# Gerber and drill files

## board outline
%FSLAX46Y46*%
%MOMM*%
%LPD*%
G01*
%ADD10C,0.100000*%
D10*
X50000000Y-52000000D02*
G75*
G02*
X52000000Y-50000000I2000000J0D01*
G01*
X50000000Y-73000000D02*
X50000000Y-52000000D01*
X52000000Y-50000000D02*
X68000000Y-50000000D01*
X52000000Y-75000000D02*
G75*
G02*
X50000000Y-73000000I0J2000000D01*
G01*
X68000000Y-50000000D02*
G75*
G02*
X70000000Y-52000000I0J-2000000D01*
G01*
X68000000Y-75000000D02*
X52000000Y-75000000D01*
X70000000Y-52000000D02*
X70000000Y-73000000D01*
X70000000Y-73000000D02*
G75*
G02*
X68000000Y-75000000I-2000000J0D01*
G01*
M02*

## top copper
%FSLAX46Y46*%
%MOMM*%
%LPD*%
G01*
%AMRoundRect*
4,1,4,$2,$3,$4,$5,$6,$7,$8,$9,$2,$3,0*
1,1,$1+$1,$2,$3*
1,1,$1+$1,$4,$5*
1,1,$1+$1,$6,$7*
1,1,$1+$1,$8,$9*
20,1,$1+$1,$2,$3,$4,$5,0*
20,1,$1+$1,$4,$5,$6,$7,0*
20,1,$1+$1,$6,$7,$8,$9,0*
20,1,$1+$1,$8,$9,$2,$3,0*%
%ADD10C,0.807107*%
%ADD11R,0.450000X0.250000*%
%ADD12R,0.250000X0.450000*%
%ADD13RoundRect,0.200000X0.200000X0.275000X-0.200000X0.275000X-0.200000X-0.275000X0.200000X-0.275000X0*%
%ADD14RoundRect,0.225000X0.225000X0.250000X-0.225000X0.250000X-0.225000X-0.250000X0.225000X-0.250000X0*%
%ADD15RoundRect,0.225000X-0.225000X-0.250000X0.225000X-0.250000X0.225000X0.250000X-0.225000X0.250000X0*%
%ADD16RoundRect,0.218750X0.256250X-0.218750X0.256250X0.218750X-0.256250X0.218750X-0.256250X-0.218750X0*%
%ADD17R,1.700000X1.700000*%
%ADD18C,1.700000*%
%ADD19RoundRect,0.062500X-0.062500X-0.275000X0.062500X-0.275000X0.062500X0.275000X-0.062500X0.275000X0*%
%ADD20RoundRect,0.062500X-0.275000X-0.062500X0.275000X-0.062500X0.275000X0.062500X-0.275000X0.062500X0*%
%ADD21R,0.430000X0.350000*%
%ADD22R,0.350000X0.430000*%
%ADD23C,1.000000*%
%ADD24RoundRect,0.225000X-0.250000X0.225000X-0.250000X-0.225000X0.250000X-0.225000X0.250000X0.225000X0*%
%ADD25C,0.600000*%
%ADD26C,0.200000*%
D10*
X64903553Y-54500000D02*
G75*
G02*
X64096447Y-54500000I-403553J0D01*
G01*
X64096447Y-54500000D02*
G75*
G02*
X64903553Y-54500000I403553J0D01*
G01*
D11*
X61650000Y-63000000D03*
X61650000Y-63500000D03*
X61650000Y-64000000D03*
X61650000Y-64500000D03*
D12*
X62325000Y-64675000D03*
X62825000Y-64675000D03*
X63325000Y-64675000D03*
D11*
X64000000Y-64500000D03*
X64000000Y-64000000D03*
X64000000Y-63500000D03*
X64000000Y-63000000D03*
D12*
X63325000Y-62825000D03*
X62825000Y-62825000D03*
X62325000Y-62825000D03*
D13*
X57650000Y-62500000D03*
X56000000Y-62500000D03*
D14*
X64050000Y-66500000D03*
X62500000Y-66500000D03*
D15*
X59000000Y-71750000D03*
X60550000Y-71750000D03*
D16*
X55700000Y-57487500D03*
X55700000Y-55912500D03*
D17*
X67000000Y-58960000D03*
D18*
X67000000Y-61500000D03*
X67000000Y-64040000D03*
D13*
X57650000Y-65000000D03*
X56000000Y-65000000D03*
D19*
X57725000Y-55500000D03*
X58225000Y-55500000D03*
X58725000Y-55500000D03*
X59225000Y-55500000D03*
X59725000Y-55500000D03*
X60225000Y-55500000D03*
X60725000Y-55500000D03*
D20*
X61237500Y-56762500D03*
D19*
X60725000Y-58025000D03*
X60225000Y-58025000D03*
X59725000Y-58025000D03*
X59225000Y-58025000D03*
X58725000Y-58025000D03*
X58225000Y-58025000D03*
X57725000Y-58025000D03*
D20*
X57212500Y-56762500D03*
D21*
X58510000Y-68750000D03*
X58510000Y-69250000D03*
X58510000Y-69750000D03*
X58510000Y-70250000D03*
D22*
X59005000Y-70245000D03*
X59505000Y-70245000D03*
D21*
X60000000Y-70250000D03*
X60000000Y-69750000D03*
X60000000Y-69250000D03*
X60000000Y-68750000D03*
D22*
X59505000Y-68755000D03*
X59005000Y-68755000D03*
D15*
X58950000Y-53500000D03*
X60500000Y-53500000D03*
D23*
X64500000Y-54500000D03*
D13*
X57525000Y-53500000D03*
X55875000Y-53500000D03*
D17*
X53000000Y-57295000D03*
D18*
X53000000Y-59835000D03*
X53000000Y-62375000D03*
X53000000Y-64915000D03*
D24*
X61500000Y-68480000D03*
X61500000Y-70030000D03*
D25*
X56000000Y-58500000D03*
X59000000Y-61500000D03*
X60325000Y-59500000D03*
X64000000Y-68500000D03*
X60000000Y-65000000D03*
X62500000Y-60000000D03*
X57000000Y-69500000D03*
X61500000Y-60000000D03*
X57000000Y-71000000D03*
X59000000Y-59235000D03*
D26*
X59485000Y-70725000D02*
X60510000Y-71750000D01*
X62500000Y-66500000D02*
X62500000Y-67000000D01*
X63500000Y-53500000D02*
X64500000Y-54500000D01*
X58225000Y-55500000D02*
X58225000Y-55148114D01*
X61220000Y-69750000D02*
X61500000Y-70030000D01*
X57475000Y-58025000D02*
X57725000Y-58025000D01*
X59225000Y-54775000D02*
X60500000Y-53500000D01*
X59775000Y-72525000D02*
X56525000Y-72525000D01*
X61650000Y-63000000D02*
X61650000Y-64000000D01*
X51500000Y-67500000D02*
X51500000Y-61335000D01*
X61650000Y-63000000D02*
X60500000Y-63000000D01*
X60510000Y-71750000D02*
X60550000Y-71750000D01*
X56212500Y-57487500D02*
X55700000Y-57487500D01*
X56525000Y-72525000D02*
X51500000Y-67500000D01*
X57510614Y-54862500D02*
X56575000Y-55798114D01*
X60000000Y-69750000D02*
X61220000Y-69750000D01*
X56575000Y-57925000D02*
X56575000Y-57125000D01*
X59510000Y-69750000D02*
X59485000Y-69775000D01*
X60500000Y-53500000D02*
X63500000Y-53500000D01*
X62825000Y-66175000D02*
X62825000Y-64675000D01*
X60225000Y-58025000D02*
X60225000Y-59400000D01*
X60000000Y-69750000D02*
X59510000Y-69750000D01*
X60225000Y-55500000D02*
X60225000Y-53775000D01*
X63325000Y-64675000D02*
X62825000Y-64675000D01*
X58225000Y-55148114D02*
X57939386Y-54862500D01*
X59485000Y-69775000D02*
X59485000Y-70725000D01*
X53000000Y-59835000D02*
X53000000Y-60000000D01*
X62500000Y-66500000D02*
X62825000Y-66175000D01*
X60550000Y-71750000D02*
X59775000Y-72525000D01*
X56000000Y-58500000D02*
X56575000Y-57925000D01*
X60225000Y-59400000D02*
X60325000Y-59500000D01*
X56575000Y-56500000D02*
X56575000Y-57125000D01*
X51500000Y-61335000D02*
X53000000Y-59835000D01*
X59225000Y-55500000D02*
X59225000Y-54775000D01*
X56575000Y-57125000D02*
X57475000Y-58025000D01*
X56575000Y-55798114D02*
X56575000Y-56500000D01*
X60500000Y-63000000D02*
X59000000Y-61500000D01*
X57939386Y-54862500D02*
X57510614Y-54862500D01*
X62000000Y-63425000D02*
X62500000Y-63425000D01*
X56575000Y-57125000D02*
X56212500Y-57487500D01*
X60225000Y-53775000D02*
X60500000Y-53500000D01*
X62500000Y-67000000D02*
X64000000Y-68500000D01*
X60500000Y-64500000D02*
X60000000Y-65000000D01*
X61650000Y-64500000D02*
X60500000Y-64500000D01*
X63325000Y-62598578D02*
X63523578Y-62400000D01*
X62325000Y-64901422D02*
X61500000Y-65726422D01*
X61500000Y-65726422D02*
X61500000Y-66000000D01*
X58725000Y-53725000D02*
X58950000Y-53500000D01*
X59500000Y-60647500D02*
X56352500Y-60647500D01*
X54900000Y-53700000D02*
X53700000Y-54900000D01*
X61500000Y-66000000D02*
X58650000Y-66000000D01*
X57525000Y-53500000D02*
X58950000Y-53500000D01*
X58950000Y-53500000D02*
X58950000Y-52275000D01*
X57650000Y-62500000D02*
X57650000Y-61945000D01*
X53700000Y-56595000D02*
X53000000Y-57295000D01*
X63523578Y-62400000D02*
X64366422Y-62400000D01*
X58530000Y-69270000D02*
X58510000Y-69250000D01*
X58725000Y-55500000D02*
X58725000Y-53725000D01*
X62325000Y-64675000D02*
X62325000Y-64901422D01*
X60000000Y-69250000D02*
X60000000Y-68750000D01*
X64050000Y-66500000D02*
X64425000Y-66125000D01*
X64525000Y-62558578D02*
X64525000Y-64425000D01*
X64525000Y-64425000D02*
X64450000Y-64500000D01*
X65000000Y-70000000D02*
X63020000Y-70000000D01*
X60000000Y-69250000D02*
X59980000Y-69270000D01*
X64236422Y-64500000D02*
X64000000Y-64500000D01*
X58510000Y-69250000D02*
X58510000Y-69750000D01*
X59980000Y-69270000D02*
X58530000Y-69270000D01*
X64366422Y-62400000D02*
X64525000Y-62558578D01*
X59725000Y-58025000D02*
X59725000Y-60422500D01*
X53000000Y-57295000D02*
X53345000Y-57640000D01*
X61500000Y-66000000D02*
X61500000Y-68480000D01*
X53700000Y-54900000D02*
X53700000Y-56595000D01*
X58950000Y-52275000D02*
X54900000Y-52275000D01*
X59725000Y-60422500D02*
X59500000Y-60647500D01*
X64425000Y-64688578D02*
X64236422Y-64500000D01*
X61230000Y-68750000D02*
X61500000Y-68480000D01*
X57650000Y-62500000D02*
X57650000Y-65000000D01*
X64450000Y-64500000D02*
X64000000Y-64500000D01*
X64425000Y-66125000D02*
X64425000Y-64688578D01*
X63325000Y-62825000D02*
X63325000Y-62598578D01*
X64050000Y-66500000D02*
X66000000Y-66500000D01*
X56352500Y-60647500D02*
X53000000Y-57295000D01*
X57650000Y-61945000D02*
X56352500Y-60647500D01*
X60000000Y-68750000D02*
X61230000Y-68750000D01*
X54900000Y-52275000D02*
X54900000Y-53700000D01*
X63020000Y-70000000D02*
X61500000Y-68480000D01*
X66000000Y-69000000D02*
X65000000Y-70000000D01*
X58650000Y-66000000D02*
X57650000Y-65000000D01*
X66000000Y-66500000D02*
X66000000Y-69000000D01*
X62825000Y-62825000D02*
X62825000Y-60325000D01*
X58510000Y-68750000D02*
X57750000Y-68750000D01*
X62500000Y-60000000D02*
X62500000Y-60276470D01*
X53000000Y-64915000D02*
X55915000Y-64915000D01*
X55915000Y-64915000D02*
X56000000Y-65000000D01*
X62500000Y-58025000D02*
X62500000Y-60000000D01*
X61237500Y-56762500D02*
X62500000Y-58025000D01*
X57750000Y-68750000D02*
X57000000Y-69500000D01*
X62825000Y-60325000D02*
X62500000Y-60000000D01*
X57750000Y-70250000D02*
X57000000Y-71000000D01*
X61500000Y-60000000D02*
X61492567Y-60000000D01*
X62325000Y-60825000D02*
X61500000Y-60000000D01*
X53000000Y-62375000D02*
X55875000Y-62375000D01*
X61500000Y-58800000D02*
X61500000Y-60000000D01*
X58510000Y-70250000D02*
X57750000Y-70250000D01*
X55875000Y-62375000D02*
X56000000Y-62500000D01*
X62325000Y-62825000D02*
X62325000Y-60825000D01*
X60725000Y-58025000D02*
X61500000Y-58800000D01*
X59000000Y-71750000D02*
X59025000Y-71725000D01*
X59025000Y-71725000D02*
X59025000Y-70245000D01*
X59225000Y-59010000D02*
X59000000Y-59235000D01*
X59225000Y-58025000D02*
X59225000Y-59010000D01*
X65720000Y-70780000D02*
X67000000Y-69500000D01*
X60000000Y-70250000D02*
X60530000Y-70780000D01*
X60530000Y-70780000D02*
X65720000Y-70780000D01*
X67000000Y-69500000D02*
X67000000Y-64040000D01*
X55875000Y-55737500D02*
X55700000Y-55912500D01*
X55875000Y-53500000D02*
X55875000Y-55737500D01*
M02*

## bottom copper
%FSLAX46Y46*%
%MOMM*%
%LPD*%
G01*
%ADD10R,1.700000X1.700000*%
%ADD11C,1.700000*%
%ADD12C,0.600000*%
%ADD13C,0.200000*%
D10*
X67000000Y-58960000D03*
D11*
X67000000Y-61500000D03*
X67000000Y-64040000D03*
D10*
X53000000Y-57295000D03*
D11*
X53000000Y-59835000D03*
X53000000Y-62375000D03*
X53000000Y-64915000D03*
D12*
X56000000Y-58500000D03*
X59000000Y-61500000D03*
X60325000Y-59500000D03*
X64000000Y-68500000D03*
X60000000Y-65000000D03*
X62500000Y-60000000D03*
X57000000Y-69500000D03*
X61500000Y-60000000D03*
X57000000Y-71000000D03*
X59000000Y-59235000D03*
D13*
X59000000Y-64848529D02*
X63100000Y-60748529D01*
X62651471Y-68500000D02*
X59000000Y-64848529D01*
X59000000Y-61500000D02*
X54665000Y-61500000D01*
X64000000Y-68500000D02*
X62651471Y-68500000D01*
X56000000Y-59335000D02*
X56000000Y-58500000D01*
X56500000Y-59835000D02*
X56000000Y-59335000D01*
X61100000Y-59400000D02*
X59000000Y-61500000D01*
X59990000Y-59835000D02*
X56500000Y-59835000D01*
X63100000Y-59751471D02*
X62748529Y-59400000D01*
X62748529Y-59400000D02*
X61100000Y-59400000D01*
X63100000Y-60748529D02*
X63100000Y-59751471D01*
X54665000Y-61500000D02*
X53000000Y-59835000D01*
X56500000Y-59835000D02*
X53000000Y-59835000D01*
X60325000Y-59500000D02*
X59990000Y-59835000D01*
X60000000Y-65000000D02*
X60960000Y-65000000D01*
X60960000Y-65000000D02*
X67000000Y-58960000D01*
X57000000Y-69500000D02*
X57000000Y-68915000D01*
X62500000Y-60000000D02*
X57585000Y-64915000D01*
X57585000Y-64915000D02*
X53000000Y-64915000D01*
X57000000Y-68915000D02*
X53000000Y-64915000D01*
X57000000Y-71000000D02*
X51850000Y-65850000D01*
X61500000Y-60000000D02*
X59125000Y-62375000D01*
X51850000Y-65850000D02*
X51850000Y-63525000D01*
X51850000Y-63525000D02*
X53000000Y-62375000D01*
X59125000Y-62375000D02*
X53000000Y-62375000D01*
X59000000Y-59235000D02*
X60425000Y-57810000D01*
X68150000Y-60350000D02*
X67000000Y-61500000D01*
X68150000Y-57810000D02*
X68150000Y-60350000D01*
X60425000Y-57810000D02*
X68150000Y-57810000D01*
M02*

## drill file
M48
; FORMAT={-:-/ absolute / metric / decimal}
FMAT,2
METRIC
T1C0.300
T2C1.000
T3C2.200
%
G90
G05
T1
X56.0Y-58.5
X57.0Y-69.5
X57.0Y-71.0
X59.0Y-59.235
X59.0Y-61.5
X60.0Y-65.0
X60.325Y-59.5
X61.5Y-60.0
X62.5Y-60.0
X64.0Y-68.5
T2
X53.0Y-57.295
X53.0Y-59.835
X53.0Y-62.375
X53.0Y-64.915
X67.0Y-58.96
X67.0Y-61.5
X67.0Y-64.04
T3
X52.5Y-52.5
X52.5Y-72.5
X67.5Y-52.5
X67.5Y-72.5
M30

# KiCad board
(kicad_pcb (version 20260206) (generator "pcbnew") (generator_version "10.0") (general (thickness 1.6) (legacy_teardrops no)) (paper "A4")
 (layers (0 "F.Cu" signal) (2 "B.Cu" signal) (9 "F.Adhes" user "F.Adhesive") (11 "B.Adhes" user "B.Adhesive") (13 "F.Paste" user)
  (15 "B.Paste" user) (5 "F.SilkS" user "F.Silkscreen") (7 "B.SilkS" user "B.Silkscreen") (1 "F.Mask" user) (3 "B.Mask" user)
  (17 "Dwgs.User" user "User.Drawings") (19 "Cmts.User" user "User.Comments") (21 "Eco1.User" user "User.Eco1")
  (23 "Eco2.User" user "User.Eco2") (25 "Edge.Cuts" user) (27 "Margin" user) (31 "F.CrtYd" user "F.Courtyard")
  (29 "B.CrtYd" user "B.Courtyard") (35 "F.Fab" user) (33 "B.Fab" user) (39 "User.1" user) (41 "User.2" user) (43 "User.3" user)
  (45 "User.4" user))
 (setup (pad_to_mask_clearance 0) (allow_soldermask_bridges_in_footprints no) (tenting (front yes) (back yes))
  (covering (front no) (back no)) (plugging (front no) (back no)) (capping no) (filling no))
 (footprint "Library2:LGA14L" (layer "F.Cu") (at 62.825 63.75)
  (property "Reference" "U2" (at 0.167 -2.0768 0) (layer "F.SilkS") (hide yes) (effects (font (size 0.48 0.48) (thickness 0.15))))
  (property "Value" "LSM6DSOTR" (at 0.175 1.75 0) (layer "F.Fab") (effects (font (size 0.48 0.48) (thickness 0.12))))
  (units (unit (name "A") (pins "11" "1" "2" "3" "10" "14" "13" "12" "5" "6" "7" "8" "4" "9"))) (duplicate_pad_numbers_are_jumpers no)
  (pad "1" smd rect (at -1.175 -0.75) (size 0.45 0.25) (layers "F.Cu" "F.Mask" "F.Paste") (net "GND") (solder_mask_margin 0.102))
  (pad "2" smd rect (at -1.175 -0.25) (size 0.45 0.25) (layers "F.Cu" "F.Mask" "F.Paste") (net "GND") (solder_mask_margin 0.102))
  (pad "3" smd rect (at -1.175 0.25) (size 0.45 0.25) (layers "F.Cu" "F.Mask" "F.Paste") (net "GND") (solder_mask_margin 0.102))
  (pad "4" smd rect (at -1.175 0.75) (size 0.45 0.25) (layers "F.Cu" "F.Mask" "F.Paste") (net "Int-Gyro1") (solder_mask_margin 0.102))
  (pad "5" smd rect (at -0.5 0.925) (size 0.25 0.45) (layers "F.Cu" "F.Mask" "F.Paste") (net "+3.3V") (solder_mask_margin 0.102))
  (pad "6" smd rect (at 0 0.925) (size 0.25 0.45) (layers "F.Cu" "F.Mask" "F.Paste") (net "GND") (solder_mask_margin 0.102))
  (pad "7" smd rect (at 0.5 0.925) (size 0.25 0.45) (layers "F.Cu" "F.Mask" "F.Paste") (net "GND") (solder_mask_margin 0.102))
  (pad "8" smd rect (at 1.175 0.75) (size 0.45 0.25) (layers "F.Cu" "F.Mask" "F.Paste") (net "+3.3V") (solder_mask_margin 0.102))
  (pad "9" smd rect (at 1.175 0.25) (size 0.45 0.25) (layers "F.Cu" "F.Mask" "F.Paste") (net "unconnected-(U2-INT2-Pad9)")
   (solder_mask_margin 0.102))
  (pad "10" smd rect (at 1.175 -0.25) (size 0.45 0.25) (layers "F.Cu" "F.Mask" "F.Paste") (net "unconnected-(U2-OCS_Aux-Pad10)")
   (solder_mask_margin 0.102))
  (pad "11" smd rect (at 1.175 -0.75) (size 0.45 0.25) (layers "F.Cu" "F.Mask" "F.Paste") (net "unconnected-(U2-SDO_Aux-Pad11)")
   (solder_mask_margin 0.102))
  (pad "12" smd rect (at 0.5 -0.925) (size 0.25 0.45) (layers "F.Cu" "F.Mask" "F.Paste") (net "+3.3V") (solder_mask_margin 0.102))
  (pad "13" smd rect (at 0 -0.925) (size 0.25 0.45) (layers "F.Cu" "F.Mask" "F.Paste") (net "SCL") (solder_mask_margin 0.102))
  (pad "14" smd rect (at -0.5 -0.925) (size 0.25 0.45) (layers "F.Cu" "F.Mask" "F.Paste") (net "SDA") (solder_mask_margin 0.102))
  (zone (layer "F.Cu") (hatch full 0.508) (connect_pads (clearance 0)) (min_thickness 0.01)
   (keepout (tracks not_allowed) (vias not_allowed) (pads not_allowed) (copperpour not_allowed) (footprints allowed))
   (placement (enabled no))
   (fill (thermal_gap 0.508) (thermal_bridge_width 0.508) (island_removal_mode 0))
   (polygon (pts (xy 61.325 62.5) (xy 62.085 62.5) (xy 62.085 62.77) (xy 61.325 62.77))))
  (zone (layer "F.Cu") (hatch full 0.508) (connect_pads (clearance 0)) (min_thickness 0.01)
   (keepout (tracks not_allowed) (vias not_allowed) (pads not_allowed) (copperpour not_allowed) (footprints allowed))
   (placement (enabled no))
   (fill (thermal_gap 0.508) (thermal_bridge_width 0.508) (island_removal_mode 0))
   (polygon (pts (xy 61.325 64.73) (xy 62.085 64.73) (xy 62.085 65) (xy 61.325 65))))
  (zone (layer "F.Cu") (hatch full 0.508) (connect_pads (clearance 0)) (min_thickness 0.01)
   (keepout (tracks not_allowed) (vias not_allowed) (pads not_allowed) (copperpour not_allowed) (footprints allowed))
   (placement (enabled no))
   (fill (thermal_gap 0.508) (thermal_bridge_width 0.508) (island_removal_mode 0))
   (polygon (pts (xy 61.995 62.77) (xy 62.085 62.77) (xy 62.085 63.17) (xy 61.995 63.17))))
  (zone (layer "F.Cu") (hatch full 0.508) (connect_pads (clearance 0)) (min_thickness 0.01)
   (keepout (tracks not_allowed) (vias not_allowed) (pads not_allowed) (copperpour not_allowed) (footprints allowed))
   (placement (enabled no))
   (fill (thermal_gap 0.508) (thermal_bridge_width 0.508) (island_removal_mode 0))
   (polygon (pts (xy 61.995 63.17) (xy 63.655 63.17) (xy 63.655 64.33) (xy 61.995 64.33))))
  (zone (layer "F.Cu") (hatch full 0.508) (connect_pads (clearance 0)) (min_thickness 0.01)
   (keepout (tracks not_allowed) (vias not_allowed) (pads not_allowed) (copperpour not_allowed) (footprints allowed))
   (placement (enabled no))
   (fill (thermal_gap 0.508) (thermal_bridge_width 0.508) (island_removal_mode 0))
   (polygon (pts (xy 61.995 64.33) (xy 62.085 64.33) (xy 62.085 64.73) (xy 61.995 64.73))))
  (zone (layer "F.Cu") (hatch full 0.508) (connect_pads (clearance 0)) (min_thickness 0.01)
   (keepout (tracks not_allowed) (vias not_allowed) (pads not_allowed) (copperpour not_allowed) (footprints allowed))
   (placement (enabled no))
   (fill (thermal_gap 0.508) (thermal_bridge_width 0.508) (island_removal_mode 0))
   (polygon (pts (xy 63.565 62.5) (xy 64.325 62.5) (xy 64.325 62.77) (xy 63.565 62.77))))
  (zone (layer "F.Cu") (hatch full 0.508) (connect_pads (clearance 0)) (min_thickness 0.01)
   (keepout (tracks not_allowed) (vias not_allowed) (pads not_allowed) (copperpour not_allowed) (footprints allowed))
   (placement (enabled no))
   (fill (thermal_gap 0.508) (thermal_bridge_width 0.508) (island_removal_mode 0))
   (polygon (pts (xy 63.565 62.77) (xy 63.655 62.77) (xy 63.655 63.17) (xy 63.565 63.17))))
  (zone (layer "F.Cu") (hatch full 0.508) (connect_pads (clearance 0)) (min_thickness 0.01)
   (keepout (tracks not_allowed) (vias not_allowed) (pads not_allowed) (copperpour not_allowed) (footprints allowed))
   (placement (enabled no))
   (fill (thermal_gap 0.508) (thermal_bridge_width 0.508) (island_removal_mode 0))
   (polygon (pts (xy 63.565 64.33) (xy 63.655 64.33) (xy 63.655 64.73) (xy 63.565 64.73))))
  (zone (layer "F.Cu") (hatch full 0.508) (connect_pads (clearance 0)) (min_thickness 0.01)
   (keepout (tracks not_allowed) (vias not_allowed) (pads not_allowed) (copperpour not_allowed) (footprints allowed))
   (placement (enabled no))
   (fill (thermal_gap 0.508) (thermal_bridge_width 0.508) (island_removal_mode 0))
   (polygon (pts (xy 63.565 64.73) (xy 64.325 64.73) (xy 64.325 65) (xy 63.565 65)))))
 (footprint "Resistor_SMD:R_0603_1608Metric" (layer "F.Cu") (at 56.825 62.5 180)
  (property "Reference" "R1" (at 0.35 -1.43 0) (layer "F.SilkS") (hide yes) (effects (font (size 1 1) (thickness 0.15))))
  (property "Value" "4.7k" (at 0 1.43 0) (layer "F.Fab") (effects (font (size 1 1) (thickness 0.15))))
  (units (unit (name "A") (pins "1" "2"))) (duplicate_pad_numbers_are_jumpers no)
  (pad "1" smd roundrect (at -0.825 0 180) (size 0.8 0.95) (layers "F.Cu" "F.Mask" "F.Paste") (roundrect_rratio 0.25) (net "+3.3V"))
  (pad "2" smd roundrect (at 0.825 0 180) (size 0.8 0.95) (layers "F.Cu" "F.Mask" "F.Paste") (roundrect_rratio 0.25) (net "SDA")))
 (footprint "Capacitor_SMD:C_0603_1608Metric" (layer "F.Cu") (at 63.275 66.5 180)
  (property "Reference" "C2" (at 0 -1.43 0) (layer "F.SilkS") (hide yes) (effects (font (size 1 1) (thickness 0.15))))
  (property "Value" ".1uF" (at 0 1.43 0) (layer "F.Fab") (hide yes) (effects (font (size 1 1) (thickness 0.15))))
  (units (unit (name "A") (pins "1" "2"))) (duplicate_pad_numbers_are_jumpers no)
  (pad "1" smd roundrect (at -0.775 0 180) (size 0.9 0.95) (layers "F.Cu" "F.Mask" "F.Paste") (roundrect_rratio 0.25) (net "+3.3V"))
  (pad "2" smd roundrect (at 0.775 0 180) (size 0.9 0.95) (layers "F.Cu" "F.Mask" "F.Paste") (roundrect_rratio 0.25) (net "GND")))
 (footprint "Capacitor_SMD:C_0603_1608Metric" (layer "F.Cu") (at 59.775 71.75)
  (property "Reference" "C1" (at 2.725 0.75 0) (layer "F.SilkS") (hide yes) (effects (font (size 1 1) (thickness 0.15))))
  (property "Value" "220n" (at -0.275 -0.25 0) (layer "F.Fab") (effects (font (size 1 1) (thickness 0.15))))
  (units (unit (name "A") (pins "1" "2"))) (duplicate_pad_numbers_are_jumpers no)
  (pad "1" smd roundrect (at -0.775 0) (size 0.9 0.95) (layers "F.Cu" "F.Mask" "F.Paste") (roundrect_rratio 0.25) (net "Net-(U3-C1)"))
  (pad "2" smd roundrect (at 0.775 0) (size 0.9 0.95) (layers "F.Cu" "F.Mask" "F.Paste") (roundrect_rratio 0.25) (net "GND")))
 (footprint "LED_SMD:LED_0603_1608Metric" (layer "F.Cu") (at 55.7 56.7 90)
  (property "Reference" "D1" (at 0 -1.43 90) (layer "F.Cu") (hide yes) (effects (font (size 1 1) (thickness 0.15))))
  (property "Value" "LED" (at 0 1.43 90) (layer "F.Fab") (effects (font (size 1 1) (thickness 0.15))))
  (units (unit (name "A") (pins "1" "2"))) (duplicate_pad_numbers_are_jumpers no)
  (pad "1" smd roundrect (at -0.7875 0 90) (size 0.875 0.95) (layers "F.Cu" "F.Mask" "F.Paste") (roundrect_rratio 0.25) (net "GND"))
  (pad "2" smd roundrect (at 0.7875 0 90) (size 0.875 0.95) (layers "F.Cu" "F.Mask" "F.Paste") (roundrect_rratio 0.25) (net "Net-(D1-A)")))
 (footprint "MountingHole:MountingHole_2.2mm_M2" (layer "F.Cu") (at 67.5 72.5)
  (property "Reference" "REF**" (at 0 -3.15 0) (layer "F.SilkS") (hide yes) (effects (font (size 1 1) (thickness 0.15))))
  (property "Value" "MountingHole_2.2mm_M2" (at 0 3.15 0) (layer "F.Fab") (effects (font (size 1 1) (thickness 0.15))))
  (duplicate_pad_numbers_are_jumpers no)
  (pad "" np_thru_hole circle (at 0 0) (size 2.2 2.2) (drill 2.2) (layers "*.Cu" "*.Mask")))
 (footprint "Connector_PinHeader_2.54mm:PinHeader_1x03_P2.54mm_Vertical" (layer "F.Cu") (at 67 58.96)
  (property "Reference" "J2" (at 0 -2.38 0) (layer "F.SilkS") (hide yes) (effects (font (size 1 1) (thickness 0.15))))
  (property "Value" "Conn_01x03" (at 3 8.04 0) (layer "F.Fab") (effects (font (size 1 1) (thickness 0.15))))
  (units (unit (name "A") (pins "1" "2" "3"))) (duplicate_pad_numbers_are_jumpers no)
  (pad "1" thru_hole rect (at 0 0) (size 1.7 1.7) (drill 1) (layers "*.Cu" "*.Mask") (remove_unused_layers no) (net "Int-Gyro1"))
  (pad "2" thru_hole circle (at 0 2.54) (size 1.7 1.7) (drill 1) (layers "*.Cu" "*.Mask") (remove_unused_layers no) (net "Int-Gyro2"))
  (pad "3" thru_hole circle (at 0 5.08) (size 1.7 1.7) (drill 1) (layers "*.Cu" "*.Mask") (remove_unused_layers no) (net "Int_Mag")))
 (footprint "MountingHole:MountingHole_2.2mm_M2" (layer "F.Cu") (at 52.5 52.5)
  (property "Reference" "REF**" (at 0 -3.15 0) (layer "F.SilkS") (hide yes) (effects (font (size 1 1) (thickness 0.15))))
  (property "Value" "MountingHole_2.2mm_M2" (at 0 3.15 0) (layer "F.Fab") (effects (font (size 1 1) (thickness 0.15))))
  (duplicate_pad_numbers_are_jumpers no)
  (pad "" np_thru_hole circle (at 0 0) (size 2.2 2.2) (drill 2.2) (layers "*.Cu" "*.Mask")))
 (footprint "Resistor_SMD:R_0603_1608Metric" (layer "F.Cu") (at 56.825 65 180)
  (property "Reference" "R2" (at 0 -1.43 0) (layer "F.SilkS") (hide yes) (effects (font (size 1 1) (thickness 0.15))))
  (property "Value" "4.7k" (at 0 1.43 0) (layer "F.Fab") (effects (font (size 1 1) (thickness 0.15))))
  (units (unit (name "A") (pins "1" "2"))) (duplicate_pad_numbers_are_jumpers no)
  (pad "1" smd roundrect (at -0.825 0 180) (size 0.8 0.95) (layers "F.Cu" "F.Mask" "F.Paste") (roundrect_rratio 0.25) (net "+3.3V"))
  (pad "2" smd roundrect (at 0.825 0 180) (size 0.8 0.95) (layers "F.Cu" "F.Mask" "F.Paste") (roundrect_rratio 0.25) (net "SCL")))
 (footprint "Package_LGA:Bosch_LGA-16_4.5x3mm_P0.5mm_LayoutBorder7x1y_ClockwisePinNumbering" (layer "F.Cu") (at 59.225 56.7625)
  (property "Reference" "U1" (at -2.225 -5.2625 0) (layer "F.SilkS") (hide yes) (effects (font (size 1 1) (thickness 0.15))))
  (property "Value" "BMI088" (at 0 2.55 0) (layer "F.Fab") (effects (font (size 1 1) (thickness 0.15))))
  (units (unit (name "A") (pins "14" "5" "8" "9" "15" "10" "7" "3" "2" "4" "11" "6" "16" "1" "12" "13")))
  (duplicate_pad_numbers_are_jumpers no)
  (pad "1" smd roundrect (at -1.5 -1.2625) (size 0.25 0.675) (layers "F.Cu" "F.Mask" "F.Paste") (roundrect_rratio 0.25)
   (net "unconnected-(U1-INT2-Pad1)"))
  (pad "2" smd roundrect (at -1 -1.2625) (size 0.25 0.675) (layers "F.Cu" "F.Mask" "F.Paste") (roundrect_rratio 0.25) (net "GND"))
  (pad "3" smd roundrect (at -0.5 -1.2625) (size 0.25 0.675) (layers "F.Cu" "F.Mask" "F.Paste") (roundrect_rratio 0.25) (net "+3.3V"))
  (pad "4" smd roundrect (at 0 -1.2625) (size 0.25 0.675) (layers "F.Cu" "F.Mask" "F.Paste") (roundrect_rratio 0.25) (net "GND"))
  (pad "5" smd roundrect (at 0.5 -1.2625) (size 0.25 0.675) (layers "F.Cu" "F.Mask" "F.Paste") (roundrect_rratio 0.25)
   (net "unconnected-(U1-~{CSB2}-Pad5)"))
  (pad "6" smd roundrect (at 1 -1.2625) (size 0.25 0.675) (layers "F.Cu" "F.Mask" "F.Paste") (roundrect_rratio 0.25) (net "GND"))
  (pad "7" smd roundrect (at 1.5 -1.2625) (size 0.25 0.675) (layers "F.Cu" "F.Mask" "F.Paste") (roundrect_rratio 0.25) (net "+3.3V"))
  (pad "8" smd roundrect (at 2.0125 0) (size 0.675 0.25) (layers "F.Cu" "F.Mask" "F.Paste") (roundrect_rratio 0.25) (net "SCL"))
  (pad "9" smd roundrect (at 1.5 1.2625) (size 0.25 0.675) (layers "F.Cu" "F.Mask" "F.Paste") (roundrect_rratio 0.25) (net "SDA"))
  (pad "10" smd roundrect (at 1 1.2625) (size 0.25 0.675) (layers "F.Cu" "F.Mask" "F.Paste") (roundrect_rratio 0.25) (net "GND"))
  (pad "11" smd roundrect (at 0.5 1.2625) (size 0.25 0.675) (layers "F.Cu" "F.Mask" "F.Paste") (roundrect_rratio 0.25) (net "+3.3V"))
  (pad "12" smd roundrect (at 0 1.2625) (size 0.25 0.675) (layers "F.Cu" "F.Mask" "F.Paste") (roundrect_rratio 0.25) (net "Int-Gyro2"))
  (pad "13" smd roundrect (at -0.5 1.2625) (size 0.25 0.675) (layers "F.Cu" "F.Mask" "F.Paste") (roundrect_rratio 0.25)
   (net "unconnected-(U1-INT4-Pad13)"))
  (pad "14" smd roundrect (at -1 1.2625) (size 0.25 0.675) (layers "F.Cu" "F.Mask" "F.Paste") (roundrect_rratio 0.25)
   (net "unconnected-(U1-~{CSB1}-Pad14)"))
  (pad "15" smd roundrect (at -1.5 1.2625) (size 0.25 0.675) (layers "F.Cu" "F.Mask" "F.Paste") (roundrect_rratio 0.25) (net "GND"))
  (pad "16" smd roundrect (at -2.0125 0) (size 0.675 0.25) (layers "F.Cu" "F.Mask" "F.Paste") (roundrect_rratio 0.25)
   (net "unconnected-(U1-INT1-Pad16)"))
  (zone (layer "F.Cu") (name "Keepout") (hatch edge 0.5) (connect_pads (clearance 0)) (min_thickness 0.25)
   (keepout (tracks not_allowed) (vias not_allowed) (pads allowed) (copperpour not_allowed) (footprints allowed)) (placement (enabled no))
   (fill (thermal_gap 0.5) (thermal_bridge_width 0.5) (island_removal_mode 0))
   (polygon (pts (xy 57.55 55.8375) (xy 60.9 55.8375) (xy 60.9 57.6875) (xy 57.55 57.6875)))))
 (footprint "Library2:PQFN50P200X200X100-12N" (layer "F.Cu") (at 59.255 69.5)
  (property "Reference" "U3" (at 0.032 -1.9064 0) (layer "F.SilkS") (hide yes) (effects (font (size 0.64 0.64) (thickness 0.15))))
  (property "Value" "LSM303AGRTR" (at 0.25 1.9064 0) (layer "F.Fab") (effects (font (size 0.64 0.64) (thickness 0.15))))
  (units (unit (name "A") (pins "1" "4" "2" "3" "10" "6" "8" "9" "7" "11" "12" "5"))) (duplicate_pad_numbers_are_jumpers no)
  (pad "1" smd rect (at -0.745 -0.75) (size 0.43 0.35) (layers "F.Cu" "F.Mask" "F.Paste") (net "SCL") (solder_mask_margin 0.102))
  (pad "2" smd rect (at -0.745 -0.25) (size 0.43 0.35) (layers "F.Cu" "F.Mask" "F.Paste") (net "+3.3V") (solder_mask_margin 0.102))
  (pad "3" smd rect (at -0.745 0.25) (size 0.43 0.35) (layers "F.Cu" "F.Mask" "F.Paste") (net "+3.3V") (solder_mask_margin 0.102))
  (pad "4" smd rect (at -0.745 0.75) (size 0.43 0.35) (layers "F.Cu" "F.Mask" "F.Paste") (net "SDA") (solder_mask_margin 0.102))
  (pad "5" smd rect (at -0.25 0.745) (size 0.35 0.43) (layers "F.Cu" "F.Mask" "F.Paste") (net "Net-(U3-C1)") (solder_mask_margin 0.102))
  (pad "6" smd rect (at 0.25 0.745) (size 0.35 0.43) (layers "F.Cu" "F.Mask" "F.Paste") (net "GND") (solder_mask_margin 0.102))
  (pad "7" smd rect (at 0.745 0.75) (size 0.43 0.35) (layers "F.Cu" "F.Mask" "F.Paste") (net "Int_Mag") (solder_mask_margin 0.102))
  (pad "8" smd rect (at 0.745 0.25) (size 0.43 0.35) (layers "F.Cu" "F.Mask" "F.Paste") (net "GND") (solder_mask_margin 0.102))
  (pad "9" smd rect (at 0.745 -0.25) (size 0.43 0.35) (layers "F.Cu" "F.Mask" "F.Paste") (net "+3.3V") (solder_mask_margin 0.102))
  (pad "10" smd rect (at 0.745 -0.75) (size 0.43 0.35) (layers "F.Cu" "F.Mask" "F.Paste") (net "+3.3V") (solder_mask_margin 0.102))
  (pad "11" smd rect (at 0.25 -0.745) (size 0.35 0.43) (layers "F.Cu" "F.Mask" "F.Paste") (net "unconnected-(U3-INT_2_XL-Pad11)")
   (solder_mask_margin 0.102))
  (pad "12" smd rect (at -0.25 -0.745) (size 0.35 0.43) (layers "F.Cu" "F.Mask" "F.Paste") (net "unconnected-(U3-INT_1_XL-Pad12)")
   (solder_mask_margin 0.102)))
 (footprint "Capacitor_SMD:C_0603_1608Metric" (layer "F.Cu") (at 59.725 53.5)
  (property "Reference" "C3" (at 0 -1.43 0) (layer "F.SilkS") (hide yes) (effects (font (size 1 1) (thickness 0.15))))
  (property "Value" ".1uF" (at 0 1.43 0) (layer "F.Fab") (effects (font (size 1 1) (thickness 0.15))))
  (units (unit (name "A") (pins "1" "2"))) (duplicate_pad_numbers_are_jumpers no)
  (pad "1" smd roundrect (at -0.775 0) (size 0.9 0.95) (layers "F.Cu" "F.Mask" "F.Paste") (roundrect_rratio 0.25) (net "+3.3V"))
  (pad "2" smd roundrect (at 0.775 0) (size 0.9 0.95) (layers "F.Cu" "F.Mask" "F.Paste") (roundrect_rratio 0.25) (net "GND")))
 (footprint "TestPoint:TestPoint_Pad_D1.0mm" (layer "F.Cu") (at 64.5 54.5)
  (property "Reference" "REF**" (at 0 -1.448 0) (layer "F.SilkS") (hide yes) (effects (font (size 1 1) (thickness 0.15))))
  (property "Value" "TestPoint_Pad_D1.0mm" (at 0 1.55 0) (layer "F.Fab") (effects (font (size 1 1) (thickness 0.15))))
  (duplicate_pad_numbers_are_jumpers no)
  (pad "1" smd circle (at 0 0) (size 1 1) (layers "F.Cu" "F.Mask")))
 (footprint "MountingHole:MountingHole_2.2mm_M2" (layer "F.Cu") (at 67.5 52.5)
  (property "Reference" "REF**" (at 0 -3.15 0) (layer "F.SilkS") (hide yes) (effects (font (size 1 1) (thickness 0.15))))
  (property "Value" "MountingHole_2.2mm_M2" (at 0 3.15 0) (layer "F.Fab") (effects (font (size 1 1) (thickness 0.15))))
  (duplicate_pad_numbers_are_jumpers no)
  (pad "" np_thru_hole circle (at 0 0) (size 2.2 2.2) (drill 2.2) (layers "*.Cu" "*.Mask")))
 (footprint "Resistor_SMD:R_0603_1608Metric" (layer "F.Cu") (at 56.7 53.5 180)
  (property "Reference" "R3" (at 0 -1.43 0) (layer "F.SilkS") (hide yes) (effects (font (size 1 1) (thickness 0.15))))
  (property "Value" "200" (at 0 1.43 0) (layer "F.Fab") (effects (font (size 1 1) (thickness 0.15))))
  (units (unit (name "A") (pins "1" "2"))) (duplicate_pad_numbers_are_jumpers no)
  (pad "1" smd roundrect (at -0.825 0 180) (size 0.8 0.95) (layers "F.Cu" "F.Mask" "F.Paste") (roundrect_rratio 0.25) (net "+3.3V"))
  (pad "2" smd roundrect (at 0.825 0 180) (size 0.8 0.95) (layers "F.Cu" "F.Mask" "F.Paste") (roundrect_rratio 0.25) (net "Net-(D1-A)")))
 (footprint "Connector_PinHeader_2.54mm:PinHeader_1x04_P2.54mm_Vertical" (layer "F.Cu") (at 53 57.295)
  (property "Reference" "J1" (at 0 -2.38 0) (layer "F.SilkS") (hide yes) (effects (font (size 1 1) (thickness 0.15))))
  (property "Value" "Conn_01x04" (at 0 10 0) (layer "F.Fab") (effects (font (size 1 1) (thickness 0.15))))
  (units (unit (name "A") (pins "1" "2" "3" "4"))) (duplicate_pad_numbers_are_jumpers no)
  (pad "1" thru_hole rect (at 0 0) (size 1.7 1.7) (drill 1) (layers "*.Cu" "*.Mask") (remove_unused_layers no) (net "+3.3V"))
  (pad "2" thru_hole circle (at 0 2.54) (size 1.7 1.7) (drill 1) (layers "*.Cu" "*.Mask") (remove_unused_layers no) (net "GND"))
  (pad "3" thru_hole circle (at 0 5.08) (size 1.7 1.7) (drill 1) (layers "*.Cu" "*.Mask") (remove_unused_layers no) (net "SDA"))
  (pad "4" thru_hole circle (at 0 7.62) (size 1.7 1.7) (drill 1) (layers "*.Cu" "*.Mask") (remove_unused_layers no) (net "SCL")))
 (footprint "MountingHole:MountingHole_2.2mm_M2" (layer "F.Cu") (at 52.5 72.5)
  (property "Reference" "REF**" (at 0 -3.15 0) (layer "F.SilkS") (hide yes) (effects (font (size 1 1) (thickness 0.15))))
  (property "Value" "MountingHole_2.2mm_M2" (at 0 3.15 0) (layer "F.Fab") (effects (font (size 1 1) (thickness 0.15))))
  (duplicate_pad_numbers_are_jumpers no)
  (pad "" np_thru_hole circle (at 0 0) (size 2.2 2.2) (drill 2.2) (layers "*.Cu" "*.Mask")))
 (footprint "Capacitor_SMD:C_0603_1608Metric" (layer "F.Cu") (at 61.5 69.255 -90)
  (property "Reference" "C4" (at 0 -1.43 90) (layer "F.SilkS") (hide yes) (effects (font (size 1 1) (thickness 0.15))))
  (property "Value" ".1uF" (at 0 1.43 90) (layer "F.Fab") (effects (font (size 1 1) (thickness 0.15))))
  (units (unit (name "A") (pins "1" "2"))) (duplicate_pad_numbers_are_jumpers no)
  (pad "1" smd roundrect (at -0.775 0 270) (size 0.9 0.95) (layers "F.Cu" "F.Mask" "F.Paste") (roundrect_rratio 0.25) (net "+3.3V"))
  (pad "2" smd roundrect (at 0.775 0 270) (size 0.9 0.95) (layers "F.Cu" "F.Mask" "F.Paste") (roundrect_rratio 0.25) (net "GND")))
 (gr_circle (center 64.5 54.5) (end 65 55) (stroke (width 0.2) (type solid)) (fill yes) (layer "F.Cu") (net "GND"))
 (gr_arc (start 50 52) (mid 50.585786 50.585786) (end 52 50) (stroke (width 0.1) (type default)) (layer "Edge.Cuts"))
 (gr_line (start 50 73) (end 50 52) (stroke (width 0.1) (type default)) (layer "Edge.Cuts"))
 (gr_line (start 52 50) (end 68 50) (stroke (width 0.1) (type default)) (layer "Edge.Cuts"))
 (gr_arc (start 52 75) (mid 50.585786 74.414214) (end 50 73) (stroke (width 0.1) (type default)) (layer "Edge.Cuts"))
 (gr_arc (start 68 50) (mid 69.414214 50.585786) (end 70 52) (stroke (width 0.1) (type default)) (layer "Edge.Cuts"))
 (gr_line (start 68 75) (end 52 75) (stroke (width 0.1) (type default)) (layer "Edge.Cuts"))
 (gr_line (start 70 52) (end 70 73) (stroke (width 0.1) (type default)) (layer "Edge.Cuts"))
 (gr_arc (start 70 73) (mid 69.414214 74.414214) (end 68 75) (stroke (width 0.1) (type default)) (layer "Edge.Cuts"))
 (segment (start 59.485 70.725) (end 60.51 71.75) (width 0.2) (layer "F.Cu") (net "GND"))
 (segment (start 62.5 66.5) (end 62.5 67) (width 0.2) (layer "F.Cu") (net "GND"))
 (segment (start 63.5 53.5) (end 64.5 54.5) (width 0.2) (layer "F.Cu") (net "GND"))
 (segment (start 58.225 55.5) (end 58.225 55.148114) (width 0.2) (layer "F.Cu") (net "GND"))
 (segment (start 61.22 69.75) (end 61.5 70.03) (width 0.2) (layer "F.Cu") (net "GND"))
 (segment (start 57.475 58.025) (end 57.725 58.025) (width 0.2) (layer "F.Cu") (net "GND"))
 (segment (start 59.225 54.775) (end 60.5 53.5) (width 0.2) (layer "F.Cu") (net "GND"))
 (segment (start 59.775 72.525) (end 56.525 72.525) (width 0.2) (layer "F.Cu") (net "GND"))
 (segment (start 61.65 63) (end 61.65 64) (width 0.2) (layer "F.Cu") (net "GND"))
 (segment (start 51.5 67.5) (end 51.5 61.335) (width 0.2) (layer "F.Cu") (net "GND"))
 (segment (start 61.65 63) (end 60.5 63) (width 0.2) (layer "F.Cu") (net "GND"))
 (segment (start 60.51 71.75) (end 60.55 71.75) (width 0.2) (layer "F.Cu") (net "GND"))
 (segment (start 56.2125 57.4875) (end 55.7 57.4875) (width 0.2) (layer "F.Cu") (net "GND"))
 (segment (start 56.525 72.525) (end 51.5 67.5) (width 0.2) (layer "F.Cu") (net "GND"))
 (segment (start 57.510614 54.8625) (end 56.575 55.798114) (width 0.2) (layer "F.Cu") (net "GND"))
 (segment (start 60 69.75) (end 61.22 69.75) (width 0.2) (layer "F.Cu") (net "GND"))
 (segment (start 56.575 57.925) (end 56.575 57.125) (width 0.2) (layer "F.Cu") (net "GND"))
 (segment (start 59.51 69.75) (end 59.485 69.775) (width 0.2) (layer "F.Cu") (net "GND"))
 (segment (start 60.5 53.5) (end 63.5 53.5) (width 0.2) (layer "F.Cu") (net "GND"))
 (segment (start 62.825 66.175) (end 62.825 64.675) (width 0.2) (layer "F.Cu") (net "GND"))
 (segment (start 60.225 58.025) (end 60.225 59.4) (width 0.2) (layer "F.Cu") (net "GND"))
 (segment (start 60 69.75) (end 59.51 69.75) (width 0.2) (layer "F.Cu") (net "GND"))
 (segment (start 60.225 55.5) (end 60.225 53.775) (width 0.2) (layer "F.Cu") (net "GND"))
 (segment (start 63.325 64.675) (end 62.825 64.675) (width 0.2) (layer "F.Cu") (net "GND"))
 (segment (start 58.225 55.148114) (end 57.939386 54.8625) (width 0.2) (layer "F.Cu") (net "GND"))
 (segment (start 59.485 69.775) (end 59.485 70.725) (width 0.2) (layer "F.Cu") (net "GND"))
 (segment (start 53 59.835) (end 53 60) (width 0.2) (layer "F.Cu") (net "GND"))
 (segment (start 62.5 66.5) (end 62.825 66.175) (width 0.2) (layer "F.Cu") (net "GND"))
 (segment (start 60.55 71.75) (end 59.775 72.525) (width 0.2) (layer "F.Cu") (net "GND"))
 (segment (start 56 58.5) (end 56.575 57.925) (width 0.2) (layer "F.Cu") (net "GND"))
 (segment (start 60.225 59.4) (end 60.325 59.5) (width 0.2) (layer "F.Cu") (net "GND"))
 (segment (start 56.575 56.5) (end 56.575 57.125) (width 0.2) (layer "F.Cu") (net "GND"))
 (segment (start 51.5 61.335) (end 53 59.835) (width 0.2) (layer "F.Cu") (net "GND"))
 (segment (start 59.225 55.5) (end 59.225 54.775) (width 0.2) (layer "F.Cu") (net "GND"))
 (segment (start 56.575 57.125) (end 57.475 58.025) (width 0.2) (layer "F.Cu") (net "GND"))
 (segment (start 56.575 55.798114) (end 56.575 56.5) (width 0.2) (layer "F.Cu") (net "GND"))
 (segment (start 60.5 63) (end 59 61.5) (width 0.2) (layer "F.Cu") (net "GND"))
 (segment (start 57.939386 54.8625) (end 57.510614 54.8625) (width 0.2) (layer "F.Cu") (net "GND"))
 (segment (start 62 63.425) (end 62.5 63.425) (width 0.2) (layer "F.Cu") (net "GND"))
 (segment (start 56.575 57.125) (end 56.2125 57.4875) (width 0.2) (layer "F.Cu") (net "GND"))
 (segment (start 60.225 53.775) (end 60.5 53.5) (width 0.2) (layer "F.Cu") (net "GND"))
 (segment (start 62.5 67) (end 64 68.5) (width 0.2) (layer "F.Cu") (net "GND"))
 (via (at 56 58.5) (size 0.6) (drill 0.3) (layers "F.Cu" "B.Cu") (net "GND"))
 (via (at 59 61.5) (size 0.6) (drill 0.3) (layers "F.Cu" "B.Cu") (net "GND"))
 (via (at 60.325 59.5) (size 0.6) (drill 0.3) (layers "F.Cu" "B.Cu") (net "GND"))
 (via (at 64 68.5) (size 0.6) (drill 0.3) (layers "F.Cu" "B.Cu") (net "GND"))
 (segment (start 59 64.848529) (end 63.1 60.748529) (width 0.2) (layer "B.Cu") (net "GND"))
 (segment (start 62.651471 68.5) (end 59 64.848529) (width 0.2) (layer "B.Cu") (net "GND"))
 (segment (start 59 61.5) (end 54.665 61.5) (width 0.2) (layer "B.Cu") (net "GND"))
 (segment (start 64 68.5) (end 62.651471 68.5) (width 0.2) (layer "B.Cu") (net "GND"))
 (segment (start 56 59.335) (end 56 58.5) (width 0.2) (layer "B.Cu") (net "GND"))
 (segment (start 56.5 59.835) (end 56 59.335) (width 0.2) (layer "B.Cu") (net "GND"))
 (segment (start 61.1 59.4) (end 59 61.5) (width 0.2) (layer "B.Cu") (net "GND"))
 (segment (start 59.99 59.835) (end 56.5 59.835) (width 0.2) (layer "B.Cu") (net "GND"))
 (segment (start 63.1 59.751471) (end 62.748529 59.4) (width 0.2) (layer "B.Cu") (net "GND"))
 (segment (start 62.748529 59.4) (end 61.1 59.4) (width 0.2) (layer "B.Cu") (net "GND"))
 (segment (start 63.1 60.748529) (end 63.1 59.751471) (width 0.2) (layer "B.Cu") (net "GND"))
 (segment (start 54.665 61.5) (end 53 59.835) (width 0.2) (layer "B.Cu") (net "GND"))
 (segment (start 56.5 59.835) (end 53 59.835) (width 0.2) (layer "B.Cu") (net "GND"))
 (segment (start 60.325 59.5) (end 59.99 59.835) (width 0.2) (layer "B.Cu") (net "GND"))
 (segment (start 60.5 64.5) (end 60 65) (width 0.2) (layer "F.Cu") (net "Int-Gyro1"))
 (segment (start 61.65 64.5) (end 60.5 64.5) (width 0.2) (layer "F.Cu") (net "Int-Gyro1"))
 (via (at 60 65) (size 0.6) (drill 0.3) (layers "F.Cu" "B.Cu") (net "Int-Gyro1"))
 (segment (start 60 65) (end 60.96 65) (width 0.2) (layer "B.Cu") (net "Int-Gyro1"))
 (segment (start 60.96 65) (end 67 58.96) (width 0.2) (layer "B.Cu") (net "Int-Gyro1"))
 (segment (start 63.325 62.598578) (end 63.523578 62.4) (width 0.2) (layer "F.Cu") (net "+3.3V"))
 (segment (start 62.325 64.901422) (end 61.5 65.726422) (width 0.2) (layer "F.Cu") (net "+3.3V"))
 (segment (start 61.5 65.726422) (end 61.5 66) (width 0.2) (layer "F.Cu") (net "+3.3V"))
 (segment (start 58.725 53.725) (end 58.95 53.5) (width 0.2) (layer "F.Cu") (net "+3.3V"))
 (segment (start 59.5 60.6475) (end 56.3525 60.6475) (width 0.2) (layer "F.Cu") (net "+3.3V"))
 (segment (start 54.9 53.7) (end 53.7 54.9) (width 0.2) (layer "F.Cu") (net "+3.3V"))
 (segment (start 61.5 66) (end 58.65 66) (width 0.2) (layer "F.Cu") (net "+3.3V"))
 (segment (start 57.525 53.5) (end 58.95 53.5) (width 0.2) (layer "F.Cu") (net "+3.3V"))
 (segment (start 58.95 53.5) (end 58.95 52.275) (width 0.2) (layer "F.Cu") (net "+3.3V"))
 (segment (start 57.65 62.5) (end 57.65 61.945) (width 0.2) (layer "F.Cu") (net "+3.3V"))
 (segment (start 53.7 56.595) (end 53 57.295) (width 0.2) (layer "F.Cu") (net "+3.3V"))
 (segment (start 63.523578 62.4) (end 64.366422 62.4) (width 0.2) (layer "F.Cu") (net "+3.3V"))
 (segment (start 58.53 69.27) (end 58.51 69.25) (width 0.2) (layer "F.Cu") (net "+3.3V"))
 (segment (start 58.725 55.5) (end 58.725 53.725) (width 0.2) (layer "F.Cu") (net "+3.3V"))
 (segment (start 62.325 64.675) (end 62.325 64.901422) (width 0.2) (layer "F.Cu") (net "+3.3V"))
 (segment (start 60 69.25) (end 60 68.75) (width 0.2) (layer "F.Cu") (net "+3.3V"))
 (segment (start 64.05 66.5) (end 64.425 66.125) (width 0.2) (layer "F.Cu") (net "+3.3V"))
 (segment (start 64.525 62.558578) (end 64.525 64.425) (width 0.2) (layer "F.Cu") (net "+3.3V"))
 (segment (start 64.525 64.425) (end 64.45 64.5) (width 0.2) (layer "F.Cu") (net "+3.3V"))
 (segment (start 65 70) (end 63.02 70) (width 0.2) (layer "F.Cu") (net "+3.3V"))
 (segment (start 60 69.25) (end 59.98 69.27) (width 0.2) (layer "F.Cu") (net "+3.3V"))
 (segment (start 64.236422 64.5) (end 64 64.5) (width 0.2) (layer "F.Cu") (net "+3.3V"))
 (segment (start 58.51 69.25) (end 58.51 69.75) (width 0.2) (layer "F.Cu") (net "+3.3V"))
 (segment (start 59.98 69.27) (end 58.53 69.27) (width 0.2) (layer "F.Cu") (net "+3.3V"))
 (segment (start 64.366422 62.4) (end 64.525 62.558578) (width 0.2) (layer "F.Cu") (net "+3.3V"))
 (segment (start 59.725 58.025) (end 59.725 60.4225) (width 0.2) (layer "F.Cu") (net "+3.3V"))
 (segment (start 53 57.295) (end 53.345 57.64) (width 0.2) (layer "F.Cu") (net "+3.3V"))
 (segment (start 61.5 66) (end 61.5 68.48) (width 0.2) (layer "F.Cu") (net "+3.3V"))
 (segment (start 53.7 54.9) (end 53.7 56.595) (width 0.2) (layer "F.Cu") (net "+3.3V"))
 (segment (start 58.95 52.275) (end 54.9 52.275) (width 0.2) (layer "F.Cu") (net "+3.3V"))
 (segment (start 59.725 60.4225) (end 59.5 60.6475) (width 0.2) (layer "F.Cu") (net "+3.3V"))
 (segment (start 64.425 64.688578) (end 64.236422 64.5) (width 0.2) (layer "F.Cu") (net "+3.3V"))
 (segment (start 61.23 68.75) (end 61.5 68.48) (width 0.2) (layer "F.Cu") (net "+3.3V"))
 (segment (start 57.65 62.5) (end 57.65 65) (width 0.2) (layer "F.Cu") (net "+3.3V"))
 (segment (start 64.45 64.5) (end 64 64.5) (width 0.2) (layer "F.Cu") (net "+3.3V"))
 (segment (start 64.425 66.125) (end 64.425 64.688578) (width 0.2) (layer "F.Cu") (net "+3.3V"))
 (segment (start 63.325 62.825) (end 63.325 62.598578) (width 0.2) (layer "F.Cu") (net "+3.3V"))
 (segment (start 64.05 66.5) (end 66 66.5) (width 0.2) (layer "F.Cu") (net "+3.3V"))
 (segment (start 56.3525 60.6475) (end 53 57.295) (width 0.2) (layer "F.Cu") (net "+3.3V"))
 (segment (start 57.65 61.945) (end 56.3525 60.6475) (width 0.2) (layer "F.Cu") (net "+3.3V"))
 (segment (start 60 68.75) (end 61.23 68.75) (width 0.2) (layer "F.Cu") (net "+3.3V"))
 (segment (start 54.9 52.275) (end 54.9 53.7) (width 0.2) (layer "F.Cu") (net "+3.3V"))
 (segment (start 63.02 70) (end 61.5 68.48) (width 0.2) (layer "F.Cu") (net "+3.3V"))
 (segment (start 66 69) (end 65 70) (width 0.2) (layer "F.Cu") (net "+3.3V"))
 (segment (start 58.65 66) (end 57.65 65) (width 0.2) (layer "F.Cu") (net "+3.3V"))
 (segment (start 66 66.5) (end 66 69) (width 0.2) (layer "F.Cu") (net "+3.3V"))
 (segment (start 62.825 62.825) (end 62.825 60.325) (width 0.2) (layer "F.Cu") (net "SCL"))
 (segment (start 58.51 68.75) (end 57.75 68.75) (width 0.2) (layer "F.Cu") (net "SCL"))
 (segment (start 62.5 60) (end 62.5 60.27647) (width 0.2) (layer "F.Cu") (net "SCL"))
 (segment (start 53 64.915) (end 55.915 64.915) (width 0.2) (layer "F.Cu") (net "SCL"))
 (segment (start 55.915 64.915) (end 56 65) (width 0.2) (layer "F.Cu") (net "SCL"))
 (segment (start 62.5 58.025) (end 62.5 60) (width 0.2) (layer "F.Cu") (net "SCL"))
 (segment (start 61.2375 56.7625) (end 62.5 58.025) (width 0.2) (layer "F.Cu") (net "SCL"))
 (segment (start 57.75 68.75) (end 57 69.5) (width 0.2) (layer "F.Cu") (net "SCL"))
 (segment (start 62.825 60.325) (end 62.5 60) (width 0.2) (layer "F.Cu") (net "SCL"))
 (via (at 62.5 60) (size 0.6) (drill 0.3) (layers "F.Cu" "B.Cu") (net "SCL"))
 (via (at 57 69.5) (size 0.6) (drill 0.3) (layers "F.Cu" "B.Cu") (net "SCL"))
 (segment (start 57 69.5) (end 57 68.915) (width 0.2) (layer "B.Cu") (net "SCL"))
 (segment (start 62.5 60) (end 57.585 64.915) (width 0.2) (layer "B.Cu") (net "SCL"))
 (segment (start 57.585 64.915) (end 53 64.915) (width 0.2) (layer "B.Cu") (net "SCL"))
 (segment (start 57 68.915) (end 53 64.915) (width 0.2) (layer "B.Cu") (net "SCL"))
 (segment (start 57.75 70.25) (end 57 71) (width 0.2) (layer "F.Cu") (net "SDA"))
 (segment (start 61.5 60) (end 61.492567 60) (width 0.2) (layer "F.Cu") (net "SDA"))
 (segment (start 62.325 60.825) (end 61.5 60) (width 0.2) (layer "F.Cu") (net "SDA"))
 (segment (start 53 62.375) (end 55.875 62.375) (width 0.2) (layer "F.Cu") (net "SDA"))
 (segment (start 61.5 58.8) (end 61.5 60) (width 0.2) (layer "F.Cu") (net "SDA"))
 (segment (start 58.51 70.25) (end 57.75 70.25) (width 0.2) (layer "F.Cu") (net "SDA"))
 (segment (start 55.875 62.375) (end 56 62.5) (width 0.2) (layer "F.Cu") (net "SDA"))
 (segment (start 62.325 62.825) (end 62.325 60.825) (width 0.2) (layer "F.Cu") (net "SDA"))
 (segment (start 60.725 58.025) (end 61.5 58.8) (width 0.2) (layer "F.Cu") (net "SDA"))
 (via (at 61.5 60) (size 0.6) (drill 0.3) (layers "F.Cu" "B.Cu") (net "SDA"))
 (via (at 57 71) (size 0.6) (drill 0.3) (layers "F.Cu" "B.Cu") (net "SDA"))
 (segment (start 57 71) (end 51.85 65.85) (width 0.2) (layer "B.Cu") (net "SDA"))
 (segment (start 61.5 60) (end 59.125 62.375) (width 0.2) (layer "B.Cu") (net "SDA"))
 (segment (start 51.85 65.85) (end 51.85 63.525) (width 0.2) (layer "B.Cu") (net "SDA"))
 (segment (start 51.85 63.525) (end 53 62.375) (width 0.2) (layer "B.Cu") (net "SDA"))
 (segment (start 59.125 62.375) (end 53 62.375) (width 0.2) (layer "B.Cu") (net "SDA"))
 (segment (start 59 71.75) (end 59.025 71.725) (width 0.2) (layer "F.Cu") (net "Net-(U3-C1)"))
 (segment (start 59.025 71.725) (end 59.025 70.245) (width 0.2) (layer "F.Cu") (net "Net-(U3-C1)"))
 (segment (start 59.225 59.01) (end 59 59.235) (width 0.2) (layer "F.Cu") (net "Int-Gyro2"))
 (segment (start 59.225 58.025) (end 59.225 59.01) (width 0.2) (layer "F.Cu") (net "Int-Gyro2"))
 (via (at 59 59.235) (size 0.6) (drill 0.3) (layers "F.Cu" "B.Cu") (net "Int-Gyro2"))
 (segment (start 59 59.235) (end 60.425 57.81) (width 0.2) (layer "B.Cu") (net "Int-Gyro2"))
 (segment (start 68.15 60.35) (end 67 61.5) (width 0.2) (layer "B.Cu") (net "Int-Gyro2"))
 (segment (start 68.15 57.81) (end 68.15 60.35) (width 0.2) (layer "B.Cu") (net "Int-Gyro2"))
 (segment (start 60.425 57.81) (end 68.15 57.81) (width 0.2) (layer "B.Cu") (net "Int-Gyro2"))
 (segment (start 65.72 70.78) (end 67 69.5) (width 0.2) (layer "F.Cu") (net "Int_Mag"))
 (segment (start 60 70.25) (end 60.53 70.78) (width 0.2) (layer "F.Cu") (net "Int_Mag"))
 (segment (start 60.53 70.78) (end 65.72 70.78) (width 0.2) (layer "F.Cu") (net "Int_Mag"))
 (segment (start 67 69.5) (end 67 64.04) (width 0.2) (layer "F.Cu") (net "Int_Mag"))
 (segment (start 55.875 55.7375) (end 55.7 55.9125) (width 0.2) (layer "F.Cu") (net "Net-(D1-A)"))
 (segment (start 55.875 53.5) (end 55.875 55.7375) (width 0.2) (layer "F.Cu") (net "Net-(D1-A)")))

